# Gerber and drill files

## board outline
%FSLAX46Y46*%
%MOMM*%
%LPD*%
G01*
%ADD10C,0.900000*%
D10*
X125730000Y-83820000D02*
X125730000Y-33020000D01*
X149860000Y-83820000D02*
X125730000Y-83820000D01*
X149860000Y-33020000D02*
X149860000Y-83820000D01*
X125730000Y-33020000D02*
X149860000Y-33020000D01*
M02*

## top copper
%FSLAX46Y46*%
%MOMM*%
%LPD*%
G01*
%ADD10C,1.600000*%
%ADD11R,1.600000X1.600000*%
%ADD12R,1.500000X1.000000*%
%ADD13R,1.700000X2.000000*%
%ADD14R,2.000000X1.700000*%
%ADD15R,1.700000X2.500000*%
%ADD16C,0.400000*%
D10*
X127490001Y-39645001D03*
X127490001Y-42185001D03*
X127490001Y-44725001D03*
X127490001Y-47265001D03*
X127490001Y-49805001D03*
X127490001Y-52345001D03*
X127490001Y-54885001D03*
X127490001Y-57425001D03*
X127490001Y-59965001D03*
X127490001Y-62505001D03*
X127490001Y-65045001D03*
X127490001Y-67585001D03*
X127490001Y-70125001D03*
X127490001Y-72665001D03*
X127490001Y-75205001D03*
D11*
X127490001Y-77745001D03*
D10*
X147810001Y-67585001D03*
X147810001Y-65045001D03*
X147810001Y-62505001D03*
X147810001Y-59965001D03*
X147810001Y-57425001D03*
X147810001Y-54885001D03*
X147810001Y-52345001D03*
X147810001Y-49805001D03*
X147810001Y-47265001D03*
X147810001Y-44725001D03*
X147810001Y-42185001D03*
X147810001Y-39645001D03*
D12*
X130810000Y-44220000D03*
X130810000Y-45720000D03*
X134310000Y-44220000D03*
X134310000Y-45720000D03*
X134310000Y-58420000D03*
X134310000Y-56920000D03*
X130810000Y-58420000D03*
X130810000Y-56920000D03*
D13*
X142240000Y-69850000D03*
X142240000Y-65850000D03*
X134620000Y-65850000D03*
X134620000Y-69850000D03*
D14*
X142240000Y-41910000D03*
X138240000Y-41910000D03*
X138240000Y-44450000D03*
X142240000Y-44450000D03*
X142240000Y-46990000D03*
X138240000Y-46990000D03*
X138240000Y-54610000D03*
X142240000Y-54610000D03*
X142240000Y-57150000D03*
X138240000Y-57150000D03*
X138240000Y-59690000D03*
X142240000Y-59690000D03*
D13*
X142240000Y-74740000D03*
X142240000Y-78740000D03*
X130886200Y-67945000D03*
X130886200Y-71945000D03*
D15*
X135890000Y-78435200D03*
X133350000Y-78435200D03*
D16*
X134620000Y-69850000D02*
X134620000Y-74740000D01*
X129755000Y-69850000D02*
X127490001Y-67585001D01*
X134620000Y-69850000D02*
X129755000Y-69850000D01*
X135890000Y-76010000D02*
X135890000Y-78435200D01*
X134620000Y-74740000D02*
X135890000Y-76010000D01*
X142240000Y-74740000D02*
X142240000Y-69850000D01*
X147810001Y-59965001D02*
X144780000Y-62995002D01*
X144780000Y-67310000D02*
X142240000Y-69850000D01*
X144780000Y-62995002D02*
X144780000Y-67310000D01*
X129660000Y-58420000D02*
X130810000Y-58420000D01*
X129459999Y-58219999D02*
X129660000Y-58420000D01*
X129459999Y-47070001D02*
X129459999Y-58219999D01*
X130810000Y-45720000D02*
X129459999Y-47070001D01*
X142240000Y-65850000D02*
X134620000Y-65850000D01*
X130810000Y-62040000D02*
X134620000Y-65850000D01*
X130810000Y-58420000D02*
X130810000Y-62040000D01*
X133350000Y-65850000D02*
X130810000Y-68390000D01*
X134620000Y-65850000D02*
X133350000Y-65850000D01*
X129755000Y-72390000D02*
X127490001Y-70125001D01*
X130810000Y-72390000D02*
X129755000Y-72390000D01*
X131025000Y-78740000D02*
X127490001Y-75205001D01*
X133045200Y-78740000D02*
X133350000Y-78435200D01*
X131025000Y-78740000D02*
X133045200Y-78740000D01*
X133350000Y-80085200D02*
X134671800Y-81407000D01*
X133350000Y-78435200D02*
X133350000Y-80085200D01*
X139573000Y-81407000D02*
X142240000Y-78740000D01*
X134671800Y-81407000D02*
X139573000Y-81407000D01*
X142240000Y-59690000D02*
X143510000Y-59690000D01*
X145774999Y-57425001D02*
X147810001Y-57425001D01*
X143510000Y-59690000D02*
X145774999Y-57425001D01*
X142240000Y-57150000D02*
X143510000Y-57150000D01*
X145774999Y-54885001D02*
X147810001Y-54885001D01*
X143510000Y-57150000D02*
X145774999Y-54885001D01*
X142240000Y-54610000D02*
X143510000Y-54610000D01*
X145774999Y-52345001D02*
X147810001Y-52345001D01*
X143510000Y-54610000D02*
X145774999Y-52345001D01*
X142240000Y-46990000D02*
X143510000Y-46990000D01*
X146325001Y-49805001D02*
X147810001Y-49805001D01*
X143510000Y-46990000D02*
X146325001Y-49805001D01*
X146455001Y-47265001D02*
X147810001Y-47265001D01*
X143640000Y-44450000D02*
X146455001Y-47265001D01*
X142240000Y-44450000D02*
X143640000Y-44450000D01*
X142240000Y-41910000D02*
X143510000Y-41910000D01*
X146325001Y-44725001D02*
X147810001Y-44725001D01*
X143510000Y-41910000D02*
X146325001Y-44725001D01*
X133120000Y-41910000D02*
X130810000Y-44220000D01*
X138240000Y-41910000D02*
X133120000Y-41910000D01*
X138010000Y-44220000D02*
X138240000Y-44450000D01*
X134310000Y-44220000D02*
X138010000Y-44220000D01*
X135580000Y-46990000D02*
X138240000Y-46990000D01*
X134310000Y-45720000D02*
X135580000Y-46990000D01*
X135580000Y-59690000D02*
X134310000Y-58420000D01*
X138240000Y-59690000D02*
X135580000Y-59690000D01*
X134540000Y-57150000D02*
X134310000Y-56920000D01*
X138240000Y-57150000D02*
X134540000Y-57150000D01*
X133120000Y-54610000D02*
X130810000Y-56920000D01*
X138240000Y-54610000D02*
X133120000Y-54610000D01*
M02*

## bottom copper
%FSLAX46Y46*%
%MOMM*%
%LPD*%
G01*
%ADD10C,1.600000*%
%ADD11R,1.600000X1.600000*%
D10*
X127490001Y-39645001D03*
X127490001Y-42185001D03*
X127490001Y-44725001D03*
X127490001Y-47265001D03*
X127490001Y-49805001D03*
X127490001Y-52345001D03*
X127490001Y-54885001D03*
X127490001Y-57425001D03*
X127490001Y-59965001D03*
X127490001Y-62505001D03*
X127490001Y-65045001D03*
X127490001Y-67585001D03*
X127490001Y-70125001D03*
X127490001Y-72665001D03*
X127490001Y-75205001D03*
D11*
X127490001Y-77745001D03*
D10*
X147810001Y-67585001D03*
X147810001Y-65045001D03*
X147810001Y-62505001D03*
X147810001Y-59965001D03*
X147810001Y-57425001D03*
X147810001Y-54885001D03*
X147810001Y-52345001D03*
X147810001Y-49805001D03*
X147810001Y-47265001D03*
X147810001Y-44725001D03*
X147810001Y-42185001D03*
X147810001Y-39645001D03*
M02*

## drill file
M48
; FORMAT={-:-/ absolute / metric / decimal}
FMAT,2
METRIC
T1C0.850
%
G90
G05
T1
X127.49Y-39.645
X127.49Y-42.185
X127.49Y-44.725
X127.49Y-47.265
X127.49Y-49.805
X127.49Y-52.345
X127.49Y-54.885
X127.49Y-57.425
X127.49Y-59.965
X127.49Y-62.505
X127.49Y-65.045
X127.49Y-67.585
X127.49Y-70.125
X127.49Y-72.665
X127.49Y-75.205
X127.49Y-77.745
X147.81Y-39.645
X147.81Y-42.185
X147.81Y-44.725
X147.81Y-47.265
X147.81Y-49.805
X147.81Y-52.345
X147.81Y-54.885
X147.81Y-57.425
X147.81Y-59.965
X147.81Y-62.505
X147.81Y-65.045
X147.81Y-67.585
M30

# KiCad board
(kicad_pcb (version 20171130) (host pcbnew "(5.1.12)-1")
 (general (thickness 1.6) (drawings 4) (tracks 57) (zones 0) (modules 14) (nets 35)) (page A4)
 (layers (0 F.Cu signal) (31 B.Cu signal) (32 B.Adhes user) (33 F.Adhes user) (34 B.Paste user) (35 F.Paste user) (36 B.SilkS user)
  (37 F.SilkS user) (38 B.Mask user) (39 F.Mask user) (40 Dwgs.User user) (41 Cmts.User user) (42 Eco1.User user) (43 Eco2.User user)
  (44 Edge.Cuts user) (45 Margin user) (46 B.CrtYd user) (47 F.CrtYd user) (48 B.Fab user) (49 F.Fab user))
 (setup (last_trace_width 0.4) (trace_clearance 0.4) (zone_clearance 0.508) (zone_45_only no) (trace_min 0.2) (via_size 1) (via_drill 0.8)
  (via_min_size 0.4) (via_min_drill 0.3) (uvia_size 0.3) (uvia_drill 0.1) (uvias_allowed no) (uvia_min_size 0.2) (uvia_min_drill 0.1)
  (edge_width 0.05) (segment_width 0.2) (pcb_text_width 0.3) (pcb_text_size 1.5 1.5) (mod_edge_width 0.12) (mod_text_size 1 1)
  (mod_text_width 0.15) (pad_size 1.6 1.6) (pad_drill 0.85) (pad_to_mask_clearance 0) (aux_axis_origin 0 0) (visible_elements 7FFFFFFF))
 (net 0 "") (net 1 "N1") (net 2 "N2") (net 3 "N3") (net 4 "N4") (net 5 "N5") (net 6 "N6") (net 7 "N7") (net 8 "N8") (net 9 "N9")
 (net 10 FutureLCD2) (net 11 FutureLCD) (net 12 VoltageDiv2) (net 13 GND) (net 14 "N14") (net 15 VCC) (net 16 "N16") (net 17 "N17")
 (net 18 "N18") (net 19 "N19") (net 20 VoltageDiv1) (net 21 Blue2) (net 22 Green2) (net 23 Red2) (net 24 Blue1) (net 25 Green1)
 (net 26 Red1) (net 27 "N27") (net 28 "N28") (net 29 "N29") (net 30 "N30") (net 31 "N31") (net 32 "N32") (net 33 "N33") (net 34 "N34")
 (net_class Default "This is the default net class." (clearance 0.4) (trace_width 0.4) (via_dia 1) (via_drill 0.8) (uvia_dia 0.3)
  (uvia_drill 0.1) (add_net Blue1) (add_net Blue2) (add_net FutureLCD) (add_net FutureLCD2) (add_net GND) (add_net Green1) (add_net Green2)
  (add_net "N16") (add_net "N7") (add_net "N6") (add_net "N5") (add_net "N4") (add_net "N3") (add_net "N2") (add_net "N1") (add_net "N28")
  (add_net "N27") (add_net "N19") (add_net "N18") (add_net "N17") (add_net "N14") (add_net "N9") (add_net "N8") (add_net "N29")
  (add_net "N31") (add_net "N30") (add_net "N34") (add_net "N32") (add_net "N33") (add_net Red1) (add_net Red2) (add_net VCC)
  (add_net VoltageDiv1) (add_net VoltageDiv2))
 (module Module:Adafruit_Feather (layer B.Cu) (at 127.490001 77.745001)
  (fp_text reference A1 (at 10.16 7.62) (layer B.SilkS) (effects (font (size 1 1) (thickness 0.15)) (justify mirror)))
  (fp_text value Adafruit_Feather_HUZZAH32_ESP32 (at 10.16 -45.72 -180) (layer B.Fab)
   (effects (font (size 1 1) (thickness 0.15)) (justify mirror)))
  (pad 16 thru_hole circle (at 0 -38.1 180) (size 1.6 1.6) (drill 0.85) (layers *.Cu *.Mask) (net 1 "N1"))
  (pad 15 thru_hole circle (at 0 -35.56 180) (size 1.6 1.6) (drill 0.85) (layers *.Cu *.Mask) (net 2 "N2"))
  (pad 14 thru_hole circle (at 0 -33.02 180) (size 1.6 1.6) (drill 0.85) (layers *.Cu *.Mask) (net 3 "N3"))
  (pad 13 thru_hole circle (at 0 -30.48 180) (size 1.6 1.6) (drill 0.85) (layers *.Cu *.Mask) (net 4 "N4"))
  (pad 12 thru_hole circle (at 0 -27.94 180) (size 1.6 1.6) (drill 0.85) (layers *.Cu *.Mask) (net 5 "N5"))
  (pad 11 thru_hole circle (at 0 -25.4 180) (size 1.6 1.6) (drill 0.85) (layers *.Cu *.Mask) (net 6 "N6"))
  (pad 10 thru_hole circle (at 0 -22.86 180) (size 1.6 1.6) (drill 0.85) (layers *.Cu *.Mask) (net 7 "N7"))
  (pad 9 thru_hole circle (at 0 -20.32 180) (size 1.6 1.6) (drill 0.85) (layers *.Cu *.Mask) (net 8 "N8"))
  (pad 8 thru_hole circle (at 0 -17.78 180) (size 1.6 1.6) (drill 0.85) (layers *.Cu *.Mask) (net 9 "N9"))
  (pad 7 thru_hole circle (at 0 -15.24 180) (size 1.6 1.6) (drill 0.85) (layers *.Cu *.Mask) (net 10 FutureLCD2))
  (pad 6 thru_hole circle (at 0 -12.7 180) (size 1.6 1.6) (drill 0.85) (layers *.Cu *.Mask) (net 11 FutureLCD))
  (pad 5 thru_hole circle (at 0 -10.16 180) (size 1.6 1.6) (drill 0.85) (layers *.Cu *.Mask) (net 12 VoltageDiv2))
  (pad 4 thru_hole circle (at 0 -7.62 180) (size 1.6 1.6) (drill 0.85) (layers *.Cu *.Mask) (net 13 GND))
  (pad 3 thru_hole circle (at 0 -5.08 180) (size 1.6 1.6) (drill 0.85) (layers *.Cu *.Mask) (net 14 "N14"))
  (pad 2 thru_hole circle (at 0 -2.54 180) (size 1.6 1.6) (drill 0.85) (layers *.Cu *.Mask) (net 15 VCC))
  (pad 1 thru_hole rect (at 0 0 180) (size 1.6 1.6) (drill 0.85) (layers *.Cu *.Mask) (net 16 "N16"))
  (pad 28 thru_hole circle (at 20.32 -10.16 180) (size 1.6 1.6) (drill 0.85) (layers *.Cu *.Mask) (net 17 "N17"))
  (pad 27 thru_hole circle (at 20.32 -12.7 180) (size 1.6 1.6) (drill 0.85) (layers *.Cu *.Mask) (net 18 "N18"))
  (pad 26 thru_hole circle (at 20.32 -15.24 180) (size 1.6 1.6) (drill 0.85) (layers *.Cu *.Mask) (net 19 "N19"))
  (pad 25 thru_hole circle (at 20.32 -17.78 180) (size 1.6 1.6) (drill 0.85) (layers *.Cu *.Mask) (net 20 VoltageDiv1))
  (pad 24 thru_hole circle (at 20.32 -20.32 180) (size 1.6 1.6) (drill 0.85) (layers *.Cu *.Mask) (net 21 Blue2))
  (pad 23 thru_hole circle (at 20.32 -22.86 180) (size 1.6 1.6) (drill 0.85) (layers *.Cu *.Mask) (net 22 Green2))
  (pad 22 thru_hole circle (at 20.32 -25.4 180) (size 1.6 1.6) (drill 0.85) (layers *.Cu *.Mask) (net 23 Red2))
  (pad 21 thru_hole circle (at 20.32 -27.94 180) (size 1.6 1.6) (drill 0.85) (layers *.Cu *.Mask) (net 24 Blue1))
  (pad 20 thru_hole circle (at 20.32 -30.48 180) (size 1.6 1.6) (drill 0.85) (layers *.Cu *.Mask) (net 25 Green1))
  (pad 19 thru_hole circle (at 20.32 -33.02 180) (size 1.6 1.6) (drill 0.85) (layers *.Cu *.Mask) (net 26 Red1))
  (pad 18 thru_hole circle (at 20.32 -35.56 180) (size 1.6 1.6) (drill 0.85) (layers *.Cu *.Mask) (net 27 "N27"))
  (pad 17 thru_hole circle (at 20.32 -38.1 180) (size 1.6 1.6) (drill 0.85) (layers *.Cu *.Mask) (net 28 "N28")))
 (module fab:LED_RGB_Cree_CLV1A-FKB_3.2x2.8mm (layer F.Cu) (at 132.56 44.97)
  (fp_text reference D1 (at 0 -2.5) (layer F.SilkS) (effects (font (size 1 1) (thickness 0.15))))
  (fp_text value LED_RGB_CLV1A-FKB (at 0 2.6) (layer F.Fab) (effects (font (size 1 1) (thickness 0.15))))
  (pad 1 smd rect (at -1.75 -0.75 180) (size 1.5 1) (layers F.Cu F.Paste F.Mask) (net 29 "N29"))
  (pad 2 smd rect (at -1.75 0.75 180) (size 1.5 1) (layers F.Cu F.Paste F.Mask) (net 13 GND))
  (pad 4 smd rect (at 1.75 -0.75 180) (size 1.5 1) (layers F.Cu F.Paste F.Mask) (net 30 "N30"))
  (pad 3 smd rect (at 1.75 0.75 180) (size 1.5 1) (layers F.Cu F.Paste F.Mask) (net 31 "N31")))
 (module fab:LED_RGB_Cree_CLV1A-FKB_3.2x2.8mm (layer F.Cu) (at 132.56 57.67)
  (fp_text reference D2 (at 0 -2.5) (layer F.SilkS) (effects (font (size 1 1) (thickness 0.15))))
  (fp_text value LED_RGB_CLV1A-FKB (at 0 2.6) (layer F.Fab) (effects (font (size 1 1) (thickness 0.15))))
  (pad 3 smd rect (at 1.75 0.75 180) (size 1.5 1) (layers F.Cu F.Paste F.Mask) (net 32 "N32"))
  (pad 4 smd rect (at 1.75 -0.75 180) (size 1.5 1) (layers F.Cu F.Paste F.Mask) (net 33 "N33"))
  (pad 2 smd rect (at -1.75 0.75 180) (size 1.5 1) (layers F.Cu F.Paste F.Mask) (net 13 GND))
  (pad 1 smd rect (at -1.75 -0.75 180) (size 1.5 1) (layers F.Cu F.Paste F.Mask) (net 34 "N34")))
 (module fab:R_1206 (layer F.Cu) (at 142.24 67.85 270)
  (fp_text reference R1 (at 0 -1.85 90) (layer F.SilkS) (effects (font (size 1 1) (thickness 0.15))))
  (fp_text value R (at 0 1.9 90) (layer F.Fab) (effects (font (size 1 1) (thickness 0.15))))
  (pad 2 smd rect (at 2 0 270) (size 2 1.7) (layers F.Cu F.Paste F.Mask) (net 20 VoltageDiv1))
  (pad 1 smd rect (at -2 0 270) (size 2 1.7) (layers F.Cu F.Paste F.Mask) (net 13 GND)))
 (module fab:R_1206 (layer F.Cu) (at 134.62 67.85 270)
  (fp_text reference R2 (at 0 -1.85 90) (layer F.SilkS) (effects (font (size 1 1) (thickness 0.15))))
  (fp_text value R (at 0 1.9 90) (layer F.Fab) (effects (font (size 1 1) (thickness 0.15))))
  (pad 1 smd rect (at -2 0 270) (size 2 1.7) (layers F.Cu F.Paste F.Mask) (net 13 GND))
  (pad 2 smd rect (at 2 0 270) (size 2 1.7) (layers F.Cu F.Paste F.Mask) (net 12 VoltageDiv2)))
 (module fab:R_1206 (layer F.Cu) (at 140.24 41.91)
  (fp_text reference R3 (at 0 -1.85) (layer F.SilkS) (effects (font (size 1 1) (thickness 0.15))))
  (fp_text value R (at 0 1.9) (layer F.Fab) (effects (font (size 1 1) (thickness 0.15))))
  (pad 2 smd rect (at 2 0) (size 2 1.7) (layers F.Cu F.Paste F.Mask) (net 26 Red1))
  (pad 1 smd rect (at -2 0) (size 2 1.7) (layers F.Cu F.Paste F.Mask) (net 29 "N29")))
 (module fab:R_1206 (layer F.Cu) (at 140.24 44.45)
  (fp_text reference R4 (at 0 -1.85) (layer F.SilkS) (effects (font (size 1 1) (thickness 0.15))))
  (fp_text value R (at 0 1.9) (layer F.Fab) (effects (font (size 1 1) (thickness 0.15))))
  (pad 1 smd rect (at -2 0) (size 2 1.7) (layers F.Cu F.Paste F.Mask) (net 30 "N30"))
  (pad 2 smd rect (at 2 0) (size 2 1.7) (layers F.Cu F.Paste F.Mask) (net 25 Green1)))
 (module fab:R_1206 (layer F.Cu) (at 140.24 46.99)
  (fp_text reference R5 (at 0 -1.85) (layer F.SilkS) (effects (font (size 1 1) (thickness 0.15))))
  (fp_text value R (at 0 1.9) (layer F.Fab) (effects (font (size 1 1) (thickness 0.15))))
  (pad 2 smd rect (at 2 0) (size 2 1.7) (layers F.Cu F.Paste F.Mask) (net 24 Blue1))
  (pad 1 smd rect (at -2 0) (size 2 1.7) (layers F.Cu F.Paste F.Mask) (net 31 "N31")))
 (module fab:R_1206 (layer F.Cu) (at 140.24 54.61)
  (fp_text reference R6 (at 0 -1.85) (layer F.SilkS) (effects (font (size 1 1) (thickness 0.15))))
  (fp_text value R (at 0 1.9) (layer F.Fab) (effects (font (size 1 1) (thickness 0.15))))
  (pad 1 smd rect (at -2 0) (size 2 1.7) (layers F.Cu F.Paste F.Mask) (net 34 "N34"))
  (pad 2 smd rect (at 2 0) (size 2 1.7) (layers F.Cu F.Paste F.Mask) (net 23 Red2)))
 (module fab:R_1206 (layer F.Cu) (at 140.24 57.15)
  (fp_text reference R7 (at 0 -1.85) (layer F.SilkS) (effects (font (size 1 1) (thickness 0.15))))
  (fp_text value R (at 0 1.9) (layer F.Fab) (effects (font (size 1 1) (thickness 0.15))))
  (pad 2 smd rect (at 2 0) (size 2 1.7) (layers F.Cu F.Paste F.Mask) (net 22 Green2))
  (pad 1 smd rect (at -2 0) (size 2 1.7) (layers F.Cu F.Paste F.Mask) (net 33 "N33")))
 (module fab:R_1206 (layer F.Cu) (at 140.24 59.69)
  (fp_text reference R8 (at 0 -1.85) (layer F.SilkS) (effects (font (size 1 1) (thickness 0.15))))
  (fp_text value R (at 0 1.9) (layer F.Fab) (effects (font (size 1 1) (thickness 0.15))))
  (pad 1 smd rect (at -2 0) (size 2 1.7) (layers F.Cu F.Paste F.Mask) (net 32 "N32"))
  (pad 2 smd rect (at 2 0) (size 2 1.7) (layers F.Cu F.Paste F.Mask) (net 21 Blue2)))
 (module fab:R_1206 (layer F.Cu) (at 142.24 76.74 270)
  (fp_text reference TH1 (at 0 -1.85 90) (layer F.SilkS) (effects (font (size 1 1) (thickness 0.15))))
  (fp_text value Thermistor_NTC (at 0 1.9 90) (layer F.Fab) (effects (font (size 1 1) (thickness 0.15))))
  (pad 1 smd rect (at -2 0 270) (size 2 1.7) (layers F.Cu F.Paste F.Mask) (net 20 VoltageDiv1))
  (pad 2 smd rect (at 2 0 270) (size 2 1.7) (layers F.Cu F.Paste F.Mask) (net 15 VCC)))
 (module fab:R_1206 (layer F.Cu) (at 130.8862 69.945 90)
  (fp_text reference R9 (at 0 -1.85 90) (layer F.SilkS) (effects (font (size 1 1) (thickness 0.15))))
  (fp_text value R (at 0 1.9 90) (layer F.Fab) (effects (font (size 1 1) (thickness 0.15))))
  (pad 2 smd rect (at 2 0 90) (size 2 1.7) (layers F.Cu F.Paste F.Mask) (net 13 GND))
  (pad 1 smd rect (at -2 0 90) (size 2 1.7) (layers F.Cu F.Paste F.Mask) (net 13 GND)))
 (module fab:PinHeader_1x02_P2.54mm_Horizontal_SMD (layer F.Cu) (at 135.89 78.4352 270)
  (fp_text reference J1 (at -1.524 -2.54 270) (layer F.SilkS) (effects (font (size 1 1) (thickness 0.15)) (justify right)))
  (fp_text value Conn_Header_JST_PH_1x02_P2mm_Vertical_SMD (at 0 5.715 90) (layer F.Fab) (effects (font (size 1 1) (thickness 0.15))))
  (pad 1 smd rect (at 0 0 270) (size 2.5 1.7) (layers F.Cu F.Paste F.Mask) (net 12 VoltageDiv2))
  (pad 2 smd rect (at 0 2.54 270) (size 2.5 1.7) (layers F.Cu F.Paste F.Mask) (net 15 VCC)))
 (gr_line (start 125.73 83.82) (end 125.73 33.02) (layer Edge.Cuts) (width 0.9))
 (gr_line (start 149.86 83.82) (end 125.73 83.82) (layer Edge.Cuts) (width 0.9))
 (gr_line (start 149.86 33.02) (end 149.86 83.82) (layer Edge.Cuts) (width 0.9))
 (gr_line (start 125.73 33.02) (end 149.86 33.02) (layer Edge.Cuts) (width 0.9))
 (segment (start 134.62 69.85) (end 134.62 74.74) (width 0.4) (layer F.Cu) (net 12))
 (segment (start 129.755 69.85) (end 127.490001 67.585001) (width 0.4) (layer F.Cu) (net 12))
 (segment (start 134.62 69.85) (end 129.755 69.85) (width 0.4) (layer F.Cu) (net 12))
 (segment (start 135.89 76.01) (end 135.89 78.4352) (width 0.4) (layer F.Cu) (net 12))
 (segment (start 134.62 74.74) (end 135.89 76.01) (width 0.4) (layer F.Cu) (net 12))
 (segment (start 142.24 74.74) (end 142.24 69.85) (width 0.4) (layer F.Cu) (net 20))
 (segment (start 147.810001 59.965001) (end 144.78 62.995002) (width 0.4) (layer F.Cu) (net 20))
 (segment (start 144.78 67.31) (end 142.24 69.85) (width 0.4) (layer F.Cu) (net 20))
 (segment (start 144.78 62.995002) (end 144.78 67.31) (width 0.4) (layer F.Cu) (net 20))
 (segment (start 129.66 58.42) (end 130.81 58.42) (width 0.4) (layer F.Cu) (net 13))
 (segment (start 129.459999 58.219999) (end 129.66 58.42) (width 0.4) (layer F.Cu) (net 13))
 (segment (start 129.459999 47.070001) (end 129.459999 58.219999) (width 0.4) (layer F.Cu) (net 13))
 (segment (start 130.81 45.72) (end 129.459999 47.070001) (width 0.4) (layer F.Cu) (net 13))
 (segment (start 142.24 65.85) (end 134.62 65.85) (width 0.4) (layer F.Cu) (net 13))
 (segment (start 130.81 62.04) (end 134.62 65.85) (width 0.4) (layer F.Cu) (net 13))
 (segment (start 130.81 58.42) (end 130.81 62.04) (width 0.4) (layer F.Cu) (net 13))
 (segment (start 133.35 65.85) (end 130.81 68.39) (width 0.4) (layer F.Cu) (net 13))
 (segment (start 134.62 65.85) (end 133.35 65.85) (width 0.4) (layer F.Cu) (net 13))
 (segment (start 129.755 72.39) (end 127.490001 70.125001) (width 0.4) (layer F.Cu) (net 13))
 (segment (start 130.81 72.39) (end 129.755 72.39) (width 0.4) (layer F.Cu) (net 13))
 (segment (start 131.025 78.74) (end 127.490001 75.205001) (width 0.4) (layer F.Cu) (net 15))
 (segment (start 133.0452 78.74) (end 133.35 78.4352) (width 0.4) (layer F.Cu) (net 15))
 (segment (start 131.025 78.74) (end 133.0452 78.74) (width 0.4) (layer F.Cu) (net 15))
 (segment (start 133.35 80.0852) (end 134.6718 81.407) (width 0.4) (layer F.Cu) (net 15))
 (segment (start 133.35 78.4352) (end 133.35 80.0852) (width 0.4) (layer F.Cu) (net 15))
 (segment (start 139.573 81.407) (end 142.24 78.74) (width 0.4) (layer F.Cu) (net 15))
 (segment (start 134.6718 81.407) (end 139.573 81.407) (width 0.4) (layer F.Cu) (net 15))
 (segment (start 142.24 59.69) (end 143.51 59.69) (width 0.4) (layer F.Cu) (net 21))
 (segment (start 145.774999 57.425001) (end 147.810001 57.425001) (width 0.4) (layer F.Cu) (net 21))
 (segment (start 143.51 59.69) (end 145.774999 57.425001) (width 0.4) (layer F.Cu) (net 21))
 (segment (start 142.24 57.15) (end 143.51 57.15) (width 0.4) (layer F.Cu) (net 22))
 (segment (start 145.774999 54.885001) (end 147.810001 54.885001) (width 0.4) (layer F.Cu) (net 22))
 (segment (start 143.51 57.15) (end 145.774999 54.885001) (width 0.4) (layer F.Cu) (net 22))
 (segment (start 142.24 54.61) (end 143.51 54.61) (width 0.4) (layer F.Cu) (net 23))
 (segment (start 145.774999 52.345001) (end 147.810001 52.345001) (width 0.4) (layer F.Cu) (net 23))
 (segment (start 143.51 54.61) (end 145.774999 52.345001) (width 0.4) (layer F.Cu) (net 23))
 (segment (start 142.24 46.99) (end 143.51 46.99) (width 0.4) (layer F.Cu) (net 24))
 (segment (start 146.325001 49.805001) (end 147.810001 49.805001) (width 0.4) (layer F.Cu) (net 24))
 (segment (start 143.51 46.99) (end 146.325001 49.805001) (width 0.4) (layer F.Cu) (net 24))
 (segment (start 146.455001 47.265001) (end 147.810001 47.265001) (width 0.4) (layer F.Cu) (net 25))
 (segment (start 143.64 44.45) (end 146.455001 47.265001) (width 0.4) (layer F.Cu) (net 25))
 (segment (start 142.24 44.45) (end 143.64 44.45) (width 0.4) (layer F.Cu) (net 25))
 (segment (start 142.24 41.91) (end 143.51 41.91) (width 0.4) (layer F.Cu) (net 26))
 (segment (start 146.325001 44.725001) (end 147.810001 44.725001) (width 0.4) (layer F.Cu) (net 26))
 (segment (start 143.51 41.91) (end 146.325001 44.725001) (width 0.4) (layer F.Cu) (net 26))
 (segment (start 133.12 41.91) (end 130.81 44.22) (width 0.4) (layer F.Cu) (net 29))
 (segment (start 138.24 41.91) (end 133.12 41.91) (width 0.4) (layer F.Cu) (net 29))
 (segment (start 138.01 44.22) (end 138.24 44.45) (width 0.4) (layer F.Cu) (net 30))
 (segment (start 134.31 44.22) (end 138.01 44.22) (width 0.4) (layer F.Cu) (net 30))
 (segment (start 135.58 46.99) (end 138.24 46.99) (width 0.4) (layer F.Cu) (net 31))
 (segment (start 134.31 45.72) (end 135.58 46.99) (width 0.4) (layer F.Cu) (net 31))
 (segment (start 135.58 59.69) (end 134.31 58.42) (width 0.4) (layer F.Cu) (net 32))
 (segment (start 138.24 59.69) (end 135.58 59.69) (width 0.4) (layer F.Cu) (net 32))
 (segment (start 134.54 57.15) (end 134.31 56.92) (width 0.4) (layer F.Cu) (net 33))
 (segment (start 138.24 57.15) (end 134.54 57.15) (width 0.4) (layer F.Cu) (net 33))
 (segment (start 133.12 54.61) (end 130.81 56.92) (width 0.4) (layer F.Cu) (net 34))
 (segment (start 138.24 54.61) (end 133.12 54.61) (width 0.4) (layer F.Cu) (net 34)))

